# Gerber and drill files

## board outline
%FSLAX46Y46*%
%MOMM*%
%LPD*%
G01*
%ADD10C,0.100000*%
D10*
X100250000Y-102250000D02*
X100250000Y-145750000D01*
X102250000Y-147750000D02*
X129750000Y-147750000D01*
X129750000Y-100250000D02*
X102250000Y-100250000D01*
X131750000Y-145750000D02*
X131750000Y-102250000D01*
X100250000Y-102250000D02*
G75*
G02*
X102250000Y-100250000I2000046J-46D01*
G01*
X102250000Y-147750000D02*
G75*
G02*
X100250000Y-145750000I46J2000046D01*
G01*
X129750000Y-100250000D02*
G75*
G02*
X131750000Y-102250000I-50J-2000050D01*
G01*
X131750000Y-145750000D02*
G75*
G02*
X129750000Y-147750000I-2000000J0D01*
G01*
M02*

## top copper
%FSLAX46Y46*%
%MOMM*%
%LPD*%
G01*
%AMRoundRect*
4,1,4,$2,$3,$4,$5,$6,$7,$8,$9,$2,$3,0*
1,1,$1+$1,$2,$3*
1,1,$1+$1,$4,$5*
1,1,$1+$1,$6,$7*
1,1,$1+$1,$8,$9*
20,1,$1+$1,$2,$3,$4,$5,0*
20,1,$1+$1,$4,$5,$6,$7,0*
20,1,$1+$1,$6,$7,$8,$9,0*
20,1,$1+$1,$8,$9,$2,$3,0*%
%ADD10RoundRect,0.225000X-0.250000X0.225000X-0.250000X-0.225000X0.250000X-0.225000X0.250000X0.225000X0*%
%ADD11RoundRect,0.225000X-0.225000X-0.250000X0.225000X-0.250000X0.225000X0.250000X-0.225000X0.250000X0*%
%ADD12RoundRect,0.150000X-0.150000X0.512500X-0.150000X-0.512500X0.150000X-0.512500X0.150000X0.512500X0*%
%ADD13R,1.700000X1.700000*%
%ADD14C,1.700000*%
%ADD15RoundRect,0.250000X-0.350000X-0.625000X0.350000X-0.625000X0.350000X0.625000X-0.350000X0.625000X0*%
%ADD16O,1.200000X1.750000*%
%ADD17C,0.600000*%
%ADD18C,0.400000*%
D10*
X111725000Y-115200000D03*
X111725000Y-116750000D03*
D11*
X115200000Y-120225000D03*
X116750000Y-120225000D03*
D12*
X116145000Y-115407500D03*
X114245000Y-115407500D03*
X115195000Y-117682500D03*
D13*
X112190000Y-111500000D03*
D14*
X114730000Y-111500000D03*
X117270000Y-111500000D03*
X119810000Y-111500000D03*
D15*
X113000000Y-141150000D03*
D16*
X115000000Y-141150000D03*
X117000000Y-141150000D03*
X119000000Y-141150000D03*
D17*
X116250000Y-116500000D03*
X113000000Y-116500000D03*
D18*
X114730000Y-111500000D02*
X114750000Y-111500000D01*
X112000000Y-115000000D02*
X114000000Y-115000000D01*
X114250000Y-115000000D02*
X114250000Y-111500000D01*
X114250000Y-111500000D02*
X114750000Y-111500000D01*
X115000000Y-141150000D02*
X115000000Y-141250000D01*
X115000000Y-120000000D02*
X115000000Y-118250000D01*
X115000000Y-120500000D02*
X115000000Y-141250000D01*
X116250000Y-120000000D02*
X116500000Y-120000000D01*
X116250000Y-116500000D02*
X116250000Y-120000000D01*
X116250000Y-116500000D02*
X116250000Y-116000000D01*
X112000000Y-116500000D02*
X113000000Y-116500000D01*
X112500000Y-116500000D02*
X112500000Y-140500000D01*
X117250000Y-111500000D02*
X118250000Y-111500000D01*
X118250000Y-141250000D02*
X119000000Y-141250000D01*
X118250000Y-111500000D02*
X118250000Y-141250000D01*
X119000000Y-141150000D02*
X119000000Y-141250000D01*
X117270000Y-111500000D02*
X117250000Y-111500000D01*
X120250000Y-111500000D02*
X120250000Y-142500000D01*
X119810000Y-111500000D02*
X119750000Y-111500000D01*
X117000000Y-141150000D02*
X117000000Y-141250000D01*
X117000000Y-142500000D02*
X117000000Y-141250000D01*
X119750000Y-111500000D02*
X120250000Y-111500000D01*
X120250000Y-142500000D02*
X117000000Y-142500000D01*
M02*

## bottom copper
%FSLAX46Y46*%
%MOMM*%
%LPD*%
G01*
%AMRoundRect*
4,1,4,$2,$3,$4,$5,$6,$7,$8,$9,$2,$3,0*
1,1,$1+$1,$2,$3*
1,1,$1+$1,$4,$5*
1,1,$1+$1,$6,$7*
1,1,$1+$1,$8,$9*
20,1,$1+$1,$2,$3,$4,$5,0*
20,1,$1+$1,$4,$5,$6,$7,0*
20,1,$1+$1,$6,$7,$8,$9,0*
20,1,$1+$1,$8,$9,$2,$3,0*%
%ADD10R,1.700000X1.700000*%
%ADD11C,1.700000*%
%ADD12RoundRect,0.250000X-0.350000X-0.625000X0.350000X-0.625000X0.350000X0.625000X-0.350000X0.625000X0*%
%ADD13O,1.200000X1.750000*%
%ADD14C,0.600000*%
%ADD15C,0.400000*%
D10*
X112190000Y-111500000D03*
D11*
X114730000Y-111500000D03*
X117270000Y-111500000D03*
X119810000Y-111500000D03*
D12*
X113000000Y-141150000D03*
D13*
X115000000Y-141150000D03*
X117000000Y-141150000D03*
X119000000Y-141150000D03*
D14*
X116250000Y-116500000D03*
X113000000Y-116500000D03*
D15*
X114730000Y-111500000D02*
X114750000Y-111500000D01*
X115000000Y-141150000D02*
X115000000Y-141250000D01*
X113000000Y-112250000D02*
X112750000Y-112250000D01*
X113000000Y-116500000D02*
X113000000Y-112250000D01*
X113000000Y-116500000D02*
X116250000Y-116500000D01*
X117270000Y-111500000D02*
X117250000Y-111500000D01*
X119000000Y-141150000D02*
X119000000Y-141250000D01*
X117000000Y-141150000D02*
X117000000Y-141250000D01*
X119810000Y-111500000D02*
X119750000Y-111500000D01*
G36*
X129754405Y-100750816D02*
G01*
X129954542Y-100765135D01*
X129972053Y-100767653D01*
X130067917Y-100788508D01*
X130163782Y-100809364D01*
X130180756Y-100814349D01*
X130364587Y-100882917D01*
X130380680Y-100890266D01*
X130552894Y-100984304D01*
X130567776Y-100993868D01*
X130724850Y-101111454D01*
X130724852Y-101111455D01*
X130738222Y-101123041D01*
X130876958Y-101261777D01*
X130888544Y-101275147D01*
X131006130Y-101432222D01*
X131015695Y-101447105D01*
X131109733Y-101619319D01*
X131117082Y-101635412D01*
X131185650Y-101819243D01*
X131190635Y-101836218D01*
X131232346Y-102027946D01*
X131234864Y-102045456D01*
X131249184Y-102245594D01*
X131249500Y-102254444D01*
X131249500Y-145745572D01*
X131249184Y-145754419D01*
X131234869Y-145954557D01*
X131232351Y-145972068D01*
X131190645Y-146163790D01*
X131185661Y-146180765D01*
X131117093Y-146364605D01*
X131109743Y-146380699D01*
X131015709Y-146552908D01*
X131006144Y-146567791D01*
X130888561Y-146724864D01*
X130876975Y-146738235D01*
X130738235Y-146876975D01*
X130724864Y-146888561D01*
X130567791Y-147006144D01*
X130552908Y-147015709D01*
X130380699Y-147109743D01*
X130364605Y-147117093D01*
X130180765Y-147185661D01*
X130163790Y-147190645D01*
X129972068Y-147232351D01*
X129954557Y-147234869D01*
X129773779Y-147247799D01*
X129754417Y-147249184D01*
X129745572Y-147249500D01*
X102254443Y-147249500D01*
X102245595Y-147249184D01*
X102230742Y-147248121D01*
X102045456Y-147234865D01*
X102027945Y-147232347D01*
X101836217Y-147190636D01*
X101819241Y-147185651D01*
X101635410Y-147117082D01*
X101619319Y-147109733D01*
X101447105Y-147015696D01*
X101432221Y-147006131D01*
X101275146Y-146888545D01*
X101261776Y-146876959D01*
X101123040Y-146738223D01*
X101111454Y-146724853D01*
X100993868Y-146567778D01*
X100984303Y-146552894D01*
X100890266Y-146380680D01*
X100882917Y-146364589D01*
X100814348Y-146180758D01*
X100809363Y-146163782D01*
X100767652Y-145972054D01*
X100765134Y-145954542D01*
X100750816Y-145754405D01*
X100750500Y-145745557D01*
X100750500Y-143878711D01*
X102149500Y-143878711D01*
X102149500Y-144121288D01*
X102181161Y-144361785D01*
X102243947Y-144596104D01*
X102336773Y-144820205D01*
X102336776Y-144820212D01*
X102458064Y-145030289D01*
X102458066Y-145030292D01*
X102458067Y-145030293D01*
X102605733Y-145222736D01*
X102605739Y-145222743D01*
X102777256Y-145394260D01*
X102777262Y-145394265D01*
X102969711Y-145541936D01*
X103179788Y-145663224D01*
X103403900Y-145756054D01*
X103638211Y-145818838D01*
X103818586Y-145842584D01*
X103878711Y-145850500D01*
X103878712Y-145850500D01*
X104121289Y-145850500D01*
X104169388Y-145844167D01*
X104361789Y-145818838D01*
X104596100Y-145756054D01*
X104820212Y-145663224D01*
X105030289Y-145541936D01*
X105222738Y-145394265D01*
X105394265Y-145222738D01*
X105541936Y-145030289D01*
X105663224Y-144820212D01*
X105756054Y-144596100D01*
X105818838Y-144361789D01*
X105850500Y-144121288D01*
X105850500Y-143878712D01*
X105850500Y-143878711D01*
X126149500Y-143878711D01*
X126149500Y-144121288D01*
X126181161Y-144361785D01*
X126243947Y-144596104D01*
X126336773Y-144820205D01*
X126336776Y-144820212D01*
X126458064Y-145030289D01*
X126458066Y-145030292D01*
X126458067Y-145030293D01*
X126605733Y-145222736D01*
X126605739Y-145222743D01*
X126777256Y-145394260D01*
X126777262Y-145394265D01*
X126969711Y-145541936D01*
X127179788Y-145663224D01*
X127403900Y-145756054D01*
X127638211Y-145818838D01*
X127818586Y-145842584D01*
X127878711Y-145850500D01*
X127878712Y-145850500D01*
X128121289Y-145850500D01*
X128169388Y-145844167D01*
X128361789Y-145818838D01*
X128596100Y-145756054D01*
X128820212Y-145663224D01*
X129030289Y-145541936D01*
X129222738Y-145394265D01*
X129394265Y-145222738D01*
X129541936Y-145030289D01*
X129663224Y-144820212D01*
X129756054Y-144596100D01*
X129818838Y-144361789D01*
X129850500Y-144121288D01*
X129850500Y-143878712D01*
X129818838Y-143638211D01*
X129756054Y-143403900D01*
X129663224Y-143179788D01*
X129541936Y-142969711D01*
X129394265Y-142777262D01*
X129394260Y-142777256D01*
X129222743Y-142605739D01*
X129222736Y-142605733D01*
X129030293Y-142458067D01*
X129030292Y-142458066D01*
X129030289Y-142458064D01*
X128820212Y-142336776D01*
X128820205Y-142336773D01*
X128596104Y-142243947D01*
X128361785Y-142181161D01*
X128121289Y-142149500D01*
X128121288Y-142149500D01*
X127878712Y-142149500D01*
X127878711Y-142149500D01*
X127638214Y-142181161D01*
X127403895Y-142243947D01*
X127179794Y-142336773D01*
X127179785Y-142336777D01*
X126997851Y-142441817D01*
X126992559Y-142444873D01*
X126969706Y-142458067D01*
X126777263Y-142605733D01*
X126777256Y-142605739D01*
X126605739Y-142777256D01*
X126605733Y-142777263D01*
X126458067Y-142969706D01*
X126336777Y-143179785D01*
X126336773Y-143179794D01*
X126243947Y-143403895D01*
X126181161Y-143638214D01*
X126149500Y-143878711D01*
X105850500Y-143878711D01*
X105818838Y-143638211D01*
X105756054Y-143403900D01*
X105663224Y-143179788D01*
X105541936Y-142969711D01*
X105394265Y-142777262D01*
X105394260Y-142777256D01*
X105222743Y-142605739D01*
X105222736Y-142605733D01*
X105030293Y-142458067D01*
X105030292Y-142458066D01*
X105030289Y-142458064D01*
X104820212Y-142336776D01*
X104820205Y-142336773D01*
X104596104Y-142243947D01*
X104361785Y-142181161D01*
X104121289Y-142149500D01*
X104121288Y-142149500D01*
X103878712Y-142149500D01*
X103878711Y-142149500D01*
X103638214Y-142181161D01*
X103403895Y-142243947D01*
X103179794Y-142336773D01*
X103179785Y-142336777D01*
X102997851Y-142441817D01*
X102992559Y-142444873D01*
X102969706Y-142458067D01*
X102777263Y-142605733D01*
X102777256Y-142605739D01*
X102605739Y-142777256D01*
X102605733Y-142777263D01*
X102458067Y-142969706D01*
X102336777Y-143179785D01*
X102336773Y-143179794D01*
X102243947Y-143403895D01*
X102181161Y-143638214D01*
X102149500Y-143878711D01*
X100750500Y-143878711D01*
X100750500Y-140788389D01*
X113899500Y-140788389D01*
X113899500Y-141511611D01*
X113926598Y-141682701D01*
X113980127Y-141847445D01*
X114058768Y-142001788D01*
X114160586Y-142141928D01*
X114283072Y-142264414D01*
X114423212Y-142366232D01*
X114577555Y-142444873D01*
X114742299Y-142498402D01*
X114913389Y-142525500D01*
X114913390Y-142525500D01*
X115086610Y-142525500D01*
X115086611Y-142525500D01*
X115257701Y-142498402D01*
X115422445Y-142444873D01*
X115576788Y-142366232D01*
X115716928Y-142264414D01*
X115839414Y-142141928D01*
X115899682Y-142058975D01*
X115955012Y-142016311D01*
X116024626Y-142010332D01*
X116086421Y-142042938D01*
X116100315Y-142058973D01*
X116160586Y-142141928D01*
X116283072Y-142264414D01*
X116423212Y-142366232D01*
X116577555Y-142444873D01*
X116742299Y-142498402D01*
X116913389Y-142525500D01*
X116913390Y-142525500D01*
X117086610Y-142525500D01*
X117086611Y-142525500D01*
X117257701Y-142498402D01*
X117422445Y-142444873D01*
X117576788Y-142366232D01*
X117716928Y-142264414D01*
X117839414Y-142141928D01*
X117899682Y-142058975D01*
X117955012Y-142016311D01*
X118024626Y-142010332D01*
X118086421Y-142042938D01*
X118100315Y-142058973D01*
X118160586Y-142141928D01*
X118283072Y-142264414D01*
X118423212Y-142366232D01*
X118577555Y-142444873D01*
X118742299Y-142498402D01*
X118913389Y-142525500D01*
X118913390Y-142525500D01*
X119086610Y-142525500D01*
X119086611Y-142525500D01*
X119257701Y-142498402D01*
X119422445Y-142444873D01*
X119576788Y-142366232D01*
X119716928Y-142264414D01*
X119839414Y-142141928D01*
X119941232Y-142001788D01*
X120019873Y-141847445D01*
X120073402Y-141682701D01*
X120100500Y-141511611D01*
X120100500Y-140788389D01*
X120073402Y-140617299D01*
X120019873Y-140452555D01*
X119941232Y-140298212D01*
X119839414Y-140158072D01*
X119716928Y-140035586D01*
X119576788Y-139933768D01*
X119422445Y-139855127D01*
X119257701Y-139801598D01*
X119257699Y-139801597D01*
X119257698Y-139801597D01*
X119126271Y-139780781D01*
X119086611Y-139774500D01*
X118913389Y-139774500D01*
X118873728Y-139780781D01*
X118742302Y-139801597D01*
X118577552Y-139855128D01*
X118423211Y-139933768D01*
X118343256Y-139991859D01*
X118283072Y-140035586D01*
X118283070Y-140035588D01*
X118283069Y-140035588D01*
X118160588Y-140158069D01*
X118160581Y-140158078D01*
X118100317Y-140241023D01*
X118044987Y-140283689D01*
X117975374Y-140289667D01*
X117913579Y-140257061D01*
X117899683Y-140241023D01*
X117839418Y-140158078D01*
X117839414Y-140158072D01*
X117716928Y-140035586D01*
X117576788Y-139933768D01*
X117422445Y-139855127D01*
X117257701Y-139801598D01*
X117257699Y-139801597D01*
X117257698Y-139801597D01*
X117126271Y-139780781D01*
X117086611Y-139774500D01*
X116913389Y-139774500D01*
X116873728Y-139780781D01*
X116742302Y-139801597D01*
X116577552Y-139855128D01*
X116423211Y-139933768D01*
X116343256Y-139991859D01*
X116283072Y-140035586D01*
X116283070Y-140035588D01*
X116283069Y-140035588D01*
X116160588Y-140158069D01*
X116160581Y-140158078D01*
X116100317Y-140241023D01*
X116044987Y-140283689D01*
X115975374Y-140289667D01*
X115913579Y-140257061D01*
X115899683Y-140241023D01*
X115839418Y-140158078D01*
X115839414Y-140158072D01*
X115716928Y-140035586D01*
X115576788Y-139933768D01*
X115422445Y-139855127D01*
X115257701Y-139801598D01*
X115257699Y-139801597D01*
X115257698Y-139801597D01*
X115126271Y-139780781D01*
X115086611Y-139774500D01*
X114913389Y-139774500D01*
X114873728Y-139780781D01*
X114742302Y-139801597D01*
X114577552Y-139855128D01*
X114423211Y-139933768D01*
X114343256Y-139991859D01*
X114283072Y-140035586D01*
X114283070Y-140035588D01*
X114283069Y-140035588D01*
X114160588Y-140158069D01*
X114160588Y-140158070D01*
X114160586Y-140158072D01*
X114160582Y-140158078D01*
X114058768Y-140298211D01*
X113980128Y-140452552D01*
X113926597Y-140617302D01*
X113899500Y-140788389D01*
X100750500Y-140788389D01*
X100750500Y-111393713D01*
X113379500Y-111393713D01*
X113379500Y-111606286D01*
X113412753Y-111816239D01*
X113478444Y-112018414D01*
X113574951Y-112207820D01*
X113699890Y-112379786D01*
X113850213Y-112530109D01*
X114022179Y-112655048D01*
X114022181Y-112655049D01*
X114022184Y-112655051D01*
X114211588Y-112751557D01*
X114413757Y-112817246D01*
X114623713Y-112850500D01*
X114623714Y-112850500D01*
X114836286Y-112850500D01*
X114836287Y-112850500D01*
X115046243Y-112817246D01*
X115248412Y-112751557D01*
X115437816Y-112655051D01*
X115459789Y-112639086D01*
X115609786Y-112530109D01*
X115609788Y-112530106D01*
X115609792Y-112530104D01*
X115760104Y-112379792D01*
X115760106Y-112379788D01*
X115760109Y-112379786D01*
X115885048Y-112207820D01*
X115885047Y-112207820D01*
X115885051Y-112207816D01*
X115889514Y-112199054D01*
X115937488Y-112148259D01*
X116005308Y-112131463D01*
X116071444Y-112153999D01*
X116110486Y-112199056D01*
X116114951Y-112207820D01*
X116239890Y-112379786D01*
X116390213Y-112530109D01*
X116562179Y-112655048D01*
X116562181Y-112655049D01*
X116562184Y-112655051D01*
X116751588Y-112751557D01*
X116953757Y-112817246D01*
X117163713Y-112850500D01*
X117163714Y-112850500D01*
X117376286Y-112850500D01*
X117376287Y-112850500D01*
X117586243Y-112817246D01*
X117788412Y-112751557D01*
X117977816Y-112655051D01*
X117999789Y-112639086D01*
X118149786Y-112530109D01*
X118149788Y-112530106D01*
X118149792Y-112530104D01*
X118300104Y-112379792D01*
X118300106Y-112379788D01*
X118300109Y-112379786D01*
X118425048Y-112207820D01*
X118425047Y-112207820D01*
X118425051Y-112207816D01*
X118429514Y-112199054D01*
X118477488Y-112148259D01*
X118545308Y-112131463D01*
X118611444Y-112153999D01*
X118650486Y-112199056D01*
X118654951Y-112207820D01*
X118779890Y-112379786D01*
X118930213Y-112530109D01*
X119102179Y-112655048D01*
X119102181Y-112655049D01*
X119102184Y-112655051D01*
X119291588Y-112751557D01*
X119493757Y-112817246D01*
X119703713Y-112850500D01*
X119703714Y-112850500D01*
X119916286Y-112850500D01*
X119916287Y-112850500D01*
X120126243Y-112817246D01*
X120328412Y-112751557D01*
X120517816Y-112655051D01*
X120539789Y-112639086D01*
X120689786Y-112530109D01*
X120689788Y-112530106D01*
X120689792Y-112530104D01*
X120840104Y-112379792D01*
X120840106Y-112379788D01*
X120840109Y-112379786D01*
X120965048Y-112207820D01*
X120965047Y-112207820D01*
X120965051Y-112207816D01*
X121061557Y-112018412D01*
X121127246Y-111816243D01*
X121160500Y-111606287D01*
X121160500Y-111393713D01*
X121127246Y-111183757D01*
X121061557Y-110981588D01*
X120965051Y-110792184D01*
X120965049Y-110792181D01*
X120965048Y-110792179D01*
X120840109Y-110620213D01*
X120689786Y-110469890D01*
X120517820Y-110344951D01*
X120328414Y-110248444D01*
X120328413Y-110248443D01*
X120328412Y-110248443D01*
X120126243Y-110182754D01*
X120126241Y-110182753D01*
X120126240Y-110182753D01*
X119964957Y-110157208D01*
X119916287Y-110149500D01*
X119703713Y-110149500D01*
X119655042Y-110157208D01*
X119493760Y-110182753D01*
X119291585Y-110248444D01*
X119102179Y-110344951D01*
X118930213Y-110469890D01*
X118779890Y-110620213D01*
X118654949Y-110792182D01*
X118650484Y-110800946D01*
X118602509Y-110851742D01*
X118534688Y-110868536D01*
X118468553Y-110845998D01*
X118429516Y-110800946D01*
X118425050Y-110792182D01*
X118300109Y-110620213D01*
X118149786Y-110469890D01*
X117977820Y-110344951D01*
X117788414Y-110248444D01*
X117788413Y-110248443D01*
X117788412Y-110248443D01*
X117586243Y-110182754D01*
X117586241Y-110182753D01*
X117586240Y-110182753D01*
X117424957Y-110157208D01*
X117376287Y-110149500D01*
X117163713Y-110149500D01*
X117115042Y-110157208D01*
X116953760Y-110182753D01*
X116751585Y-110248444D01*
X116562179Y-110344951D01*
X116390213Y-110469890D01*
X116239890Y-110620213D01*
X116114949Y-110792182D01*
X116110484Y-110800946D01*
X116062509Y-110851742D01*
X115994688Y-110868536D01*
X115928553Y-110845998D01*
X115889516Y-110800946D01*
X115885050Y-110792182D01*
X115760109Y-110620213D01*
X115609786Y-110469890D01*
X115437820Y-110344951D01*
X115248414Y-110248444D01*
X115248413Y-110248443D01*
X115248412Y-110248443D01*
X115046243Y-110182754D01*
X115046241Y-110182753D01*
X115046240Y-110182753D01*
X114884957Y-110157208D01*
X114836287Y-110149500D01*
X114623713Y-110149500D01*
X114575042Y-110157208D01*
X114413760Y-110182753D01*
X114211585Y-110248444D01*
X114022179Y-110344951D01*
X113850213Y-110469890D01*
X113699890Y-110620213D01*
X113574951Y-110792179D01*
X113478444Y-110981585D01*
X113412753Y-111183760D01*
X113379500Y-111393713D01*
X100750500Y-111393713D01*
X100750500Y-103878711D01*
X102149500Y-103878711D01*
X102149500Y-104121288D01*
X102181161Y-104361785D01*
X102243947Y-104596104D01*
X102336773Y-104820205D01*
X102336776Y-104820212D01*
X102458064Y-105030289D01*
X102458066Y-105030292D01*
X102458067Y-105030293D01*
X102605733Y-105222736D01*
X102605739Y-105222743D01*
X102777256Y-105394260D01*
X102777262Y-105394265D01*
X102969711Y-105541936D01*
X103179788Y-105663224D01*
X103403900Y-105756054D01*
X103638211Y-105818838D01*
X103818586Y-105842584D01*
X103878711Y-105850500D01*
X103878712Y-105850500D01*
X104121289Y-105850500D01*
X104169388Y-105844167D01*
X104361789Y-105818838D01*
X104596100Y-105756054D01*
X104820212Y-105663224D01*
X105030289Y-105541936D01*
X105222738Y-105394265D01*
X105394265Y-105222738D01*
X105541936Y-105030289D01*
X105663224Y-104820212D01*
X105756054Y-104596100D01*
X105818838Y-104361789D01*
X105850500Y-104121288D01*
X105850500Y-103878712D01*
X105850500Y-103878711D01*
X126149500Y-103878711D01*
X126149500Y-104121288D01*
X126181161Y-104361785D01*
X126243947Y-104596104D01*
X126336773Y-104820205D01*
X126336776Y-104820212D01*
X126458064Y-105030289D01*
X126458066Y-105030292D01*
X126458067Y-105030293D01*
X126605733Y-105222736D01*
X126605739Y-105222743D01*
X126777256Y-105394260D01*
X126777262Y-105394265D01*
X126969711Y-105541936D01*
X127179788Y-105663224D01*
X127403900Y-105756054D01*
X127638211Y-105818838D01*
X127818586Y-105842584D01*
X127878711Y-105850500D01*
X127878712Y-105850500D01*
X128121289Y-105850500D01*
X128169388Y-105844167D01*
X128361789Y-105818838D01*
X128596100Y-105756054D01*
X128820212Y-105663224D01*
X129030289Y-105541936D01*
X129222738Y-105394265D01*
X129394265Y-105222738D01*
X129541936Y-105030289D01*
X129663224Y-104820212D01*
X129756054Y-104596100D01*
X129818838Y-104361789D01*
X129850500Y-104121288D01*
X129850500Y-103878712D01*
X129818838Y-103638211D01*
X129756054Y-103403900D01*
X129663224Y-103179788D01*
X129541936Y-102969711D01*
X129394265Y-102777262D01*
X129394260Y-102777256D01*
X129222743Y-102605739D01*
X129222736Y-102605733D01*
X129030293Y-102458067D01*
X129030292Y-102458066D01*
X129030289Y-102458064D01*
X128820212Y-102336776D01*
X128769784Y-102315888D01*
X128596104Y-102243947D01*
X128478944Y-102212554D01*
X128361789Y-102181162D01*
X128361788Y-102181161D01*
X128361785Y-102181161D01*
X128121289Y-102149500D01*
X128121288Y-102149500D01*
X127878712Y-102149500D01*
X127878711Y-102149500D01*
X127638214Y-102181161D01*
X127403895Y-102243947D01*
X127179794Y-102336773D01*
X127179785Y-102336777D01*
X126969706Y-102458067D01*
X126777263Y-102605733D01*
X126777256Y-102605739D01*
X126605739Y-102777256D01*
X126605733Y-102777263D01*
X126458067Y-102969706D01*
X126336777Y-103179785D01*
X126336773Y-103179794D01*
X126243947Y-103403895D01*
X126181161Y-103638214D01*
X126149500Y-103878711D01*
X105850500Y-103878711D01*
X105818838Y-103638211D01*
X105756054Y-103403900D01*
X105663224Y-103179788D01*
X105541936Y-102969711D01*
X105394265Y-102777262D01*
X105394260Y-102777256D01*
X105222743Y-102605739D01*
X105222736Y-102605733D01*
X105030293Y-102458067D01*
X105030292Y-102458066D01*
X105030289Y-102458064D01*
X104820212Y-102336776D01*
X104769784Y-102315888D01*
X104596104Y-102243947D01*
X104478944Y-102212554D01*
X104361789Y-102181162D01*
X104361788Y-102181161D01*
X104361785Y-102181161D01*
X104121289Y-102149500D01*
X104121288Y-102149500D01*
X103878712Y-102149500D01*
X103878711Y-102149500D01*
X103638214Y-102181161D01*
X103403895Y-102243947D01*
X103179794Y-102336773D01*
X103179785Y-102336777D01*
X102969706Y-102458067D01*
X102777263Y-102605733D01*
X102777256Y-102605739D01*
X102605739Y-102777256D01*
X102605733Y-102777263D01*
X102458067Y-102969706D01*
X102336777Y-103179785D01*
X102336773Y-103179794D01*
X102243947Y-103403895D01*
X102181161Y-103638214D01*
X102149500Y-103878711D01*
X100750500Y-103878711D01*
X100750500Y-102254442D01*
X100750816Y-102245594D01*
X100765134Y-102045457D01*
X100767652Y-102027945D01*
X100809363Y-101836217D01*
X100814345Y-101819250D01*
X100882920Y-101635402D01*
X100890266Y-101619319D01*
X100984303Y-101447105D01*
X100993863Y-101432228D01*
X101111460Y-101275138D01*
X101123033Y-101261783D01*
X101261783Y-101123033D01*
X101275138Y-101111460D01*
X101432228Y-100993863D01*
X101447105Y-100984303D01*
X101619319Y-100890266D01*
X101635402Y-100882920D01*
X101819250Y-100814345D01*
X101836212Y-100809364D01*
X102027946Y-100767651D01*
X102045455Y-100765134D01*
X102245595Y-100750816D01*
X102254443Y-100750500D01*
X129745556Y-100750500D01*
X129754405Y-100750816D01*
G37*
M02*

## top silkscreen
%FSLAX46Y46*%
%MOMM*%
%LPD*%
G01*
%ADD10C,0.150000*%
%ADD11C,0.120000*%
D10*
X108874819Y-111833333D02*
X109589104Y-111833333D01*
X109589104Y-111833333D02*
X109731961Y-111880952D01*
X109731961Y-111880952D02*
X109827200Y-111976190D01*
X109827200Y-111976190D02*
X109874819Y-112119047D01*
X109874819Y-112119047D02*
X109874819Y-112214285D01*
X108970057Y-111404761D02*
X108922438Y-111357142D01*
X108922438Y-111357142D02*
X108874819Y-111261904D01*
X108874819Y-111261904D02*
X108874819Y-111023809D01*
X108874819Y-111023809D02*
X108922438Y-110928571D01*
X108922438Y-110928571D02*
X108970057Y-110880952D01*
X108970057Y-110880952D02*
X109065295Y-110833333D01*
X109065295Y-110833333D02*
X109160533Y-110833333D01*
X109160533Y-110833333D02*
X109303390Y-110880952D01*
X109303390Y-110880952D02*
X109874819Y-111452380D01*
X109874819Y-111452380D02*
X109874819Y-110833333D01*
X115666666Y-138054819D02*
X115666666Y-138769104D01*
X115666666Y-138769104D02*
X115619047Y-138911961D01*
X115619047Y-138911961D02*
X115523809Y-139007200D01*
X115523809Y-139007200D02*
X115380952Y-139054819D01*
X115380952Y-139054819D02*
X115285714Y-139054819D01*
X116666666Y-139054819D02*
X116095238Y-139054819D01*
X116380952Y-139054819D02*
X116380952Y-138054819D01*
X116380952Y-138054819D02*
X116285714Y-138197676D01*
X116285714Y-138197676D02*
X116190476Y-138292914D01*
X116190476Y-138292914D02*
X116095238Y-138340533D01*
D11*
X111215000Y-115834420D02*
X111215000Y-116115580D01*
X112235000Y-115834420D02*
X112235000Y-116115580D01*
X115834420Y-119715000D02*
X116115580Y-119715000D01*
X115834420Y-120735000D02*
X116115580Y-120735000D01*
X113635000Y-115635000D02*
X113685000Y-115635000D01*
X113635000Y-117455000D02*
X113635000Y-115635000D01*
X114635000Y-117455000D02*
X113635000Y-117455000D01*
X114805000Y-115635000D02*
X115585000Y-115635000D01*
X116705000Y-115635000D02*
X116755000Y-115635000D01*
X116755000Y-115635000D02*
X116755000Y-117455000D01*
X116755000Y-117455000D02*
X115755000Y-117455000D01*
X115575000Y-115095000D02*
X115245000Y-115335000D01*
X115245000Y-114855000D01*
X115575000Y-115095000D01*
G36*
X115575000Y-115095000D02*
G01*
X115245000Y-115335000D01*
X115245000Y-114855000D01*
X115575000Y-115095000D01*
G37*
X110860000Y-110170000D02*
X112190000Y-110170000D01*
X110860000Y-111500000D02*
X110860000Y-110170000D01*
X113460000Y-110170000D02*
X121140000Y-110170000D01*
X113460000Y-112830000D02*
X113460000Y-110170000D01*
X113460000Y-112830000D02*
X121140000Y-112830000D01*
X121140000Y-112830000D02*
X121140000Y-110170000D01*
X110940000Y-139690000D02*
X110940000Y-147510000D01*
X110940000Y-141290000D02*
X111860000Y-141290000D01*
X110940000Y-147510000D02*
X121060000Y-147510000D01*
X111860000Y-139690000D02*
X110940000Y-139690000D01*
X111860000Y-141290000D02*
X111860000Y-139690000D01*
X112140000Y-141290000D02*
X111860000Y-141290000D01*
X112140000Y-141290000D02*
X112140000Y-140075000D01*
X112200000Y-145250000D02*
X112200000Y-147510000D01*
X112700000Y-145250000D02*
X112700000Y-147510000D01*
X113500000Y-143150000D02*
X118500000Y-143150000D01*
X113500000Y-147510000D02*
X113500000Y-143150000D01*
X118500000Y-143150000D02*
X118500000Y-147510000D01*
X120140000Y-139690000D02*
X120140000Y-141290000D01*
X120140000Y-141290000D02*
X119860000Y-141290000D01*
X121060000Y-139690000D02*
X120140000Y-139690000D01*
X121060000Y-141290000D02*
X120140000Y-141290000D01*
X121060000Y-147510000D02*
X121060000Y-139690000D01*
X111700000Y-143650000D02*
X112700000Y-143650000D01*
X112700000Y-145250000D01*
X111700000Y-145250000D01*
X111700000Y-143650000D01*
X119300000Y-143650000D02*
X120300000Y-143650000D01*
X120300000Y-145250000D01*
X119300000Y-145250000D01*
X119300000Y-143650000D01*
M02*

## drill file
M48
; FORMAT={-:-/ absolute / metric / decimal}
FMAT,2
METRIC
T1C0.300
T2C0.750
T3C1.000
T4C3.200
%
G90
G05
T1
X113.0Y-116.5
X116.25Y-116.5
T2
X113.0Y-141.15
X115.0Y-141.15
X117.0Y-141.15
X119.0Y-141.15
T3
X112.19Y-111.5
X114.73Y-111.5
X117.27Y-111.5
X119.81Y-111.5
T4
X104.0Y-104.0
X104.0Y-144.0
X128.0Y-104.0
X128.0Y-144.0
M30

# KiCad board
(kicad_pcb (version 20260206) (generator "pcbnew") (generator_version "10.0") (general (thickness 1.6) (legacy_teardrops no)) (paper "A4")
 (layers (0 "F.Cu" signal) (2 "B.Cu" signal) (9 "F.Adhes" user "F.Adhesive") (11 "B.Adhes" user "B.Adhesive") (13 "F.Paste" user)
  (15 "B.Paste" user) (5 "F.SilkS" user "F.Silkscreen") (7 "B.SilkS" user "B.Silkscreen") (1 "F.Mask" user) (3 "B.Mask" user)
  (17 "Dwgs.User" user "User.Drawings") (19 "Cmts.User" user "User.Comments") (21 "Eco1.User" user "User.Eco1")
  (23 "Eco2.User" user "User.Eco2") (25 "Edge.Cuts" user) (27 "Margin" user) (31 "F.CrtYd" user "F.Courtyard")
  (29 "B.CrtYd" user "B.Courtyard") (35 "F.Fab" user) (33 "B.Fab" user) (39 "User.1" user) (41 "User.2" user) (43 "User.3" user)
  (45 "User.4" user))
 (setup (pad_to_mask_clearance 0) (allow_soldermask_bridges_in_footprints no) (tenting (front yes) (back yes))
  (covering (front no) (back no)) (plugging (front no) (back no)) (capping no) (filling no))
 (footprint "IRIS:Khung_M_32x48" (layer "F.Cu") (at 100 148)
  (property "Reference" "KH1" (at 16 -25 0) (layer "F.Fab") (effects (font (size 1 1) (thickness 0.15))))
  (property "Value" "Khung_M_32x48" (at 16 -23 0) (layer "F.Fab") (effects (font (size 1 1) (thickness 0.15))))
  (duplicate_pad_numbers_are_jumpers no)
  (fp_line (start 0.25 -45.75) (end 0.25 -2.25) (stroke (width 0.1) (type solid)) (layer "Edge.Cuts"))
  (fp_line (start 2.25 -0.25) (end 29.75 -0.25) (stroke (width 0.1) (type solid)) (layer "Edge.Cuts"))
  (fp_line (start 29.75 -47.75) (end 2.25 -47.75) (stroke (width 0.1) (type solid)) (layer "Edge.Cuts"))
  (fp_line (start 31.75 -2.25) (end 31.75 -45.75) (stroke (width 0.1) (type solid)) (layer "Edge.Cuts"))
  (fp_arc (start 0.25 -45.75) (mid 0.8358 -47.1642) (end 2.25 -47.75) (stroke (width 0.1) (type solid)) (layer "Edge.Cuts"))
  (fp_arc (start 2.25 -0.25) (mid 0.8358 -0.8358) (end 0.25 -2.25) (stroke (width 0.1) (type solid)) (layer "Edge.Cuts"))
  (fp_arc (start 29.75 -47.75) (mid 31.164199 -47.164199) (end 31.75 -45.75) (stroke (width 0.1) (type solid)) (layer "Edge.Cuts"))
  (fp_arc (start 31.75 -2.25) (mid 31.164214 -0.835786) (end 29.75 -0.25) (stroke (width 0.1) (type solid)) (layer "Edge.Cuts"))
  (pad "" np_thru_hole circle (at 4 -44) (size 3.2 3.2) (drill 3.2) (layers "*.Cu" "*.Mask"))
  (pad "" np_thru_hole circle (at 4 -4) (size 3.2 3.2) (drill 3.2) (layers "*.Cu" "*.Mask"))
  (pad "" np_thru_hole circle (at 28 -44) (size 3.2 3.2) (drill 3.2) (layers "*.Cu" "*.Mask"))
  (pad "" np_thru_hole circle (at 28 -4) (size 3.2 3.2) (drill 3.2) (layers "*.Cu" "*.Mask")))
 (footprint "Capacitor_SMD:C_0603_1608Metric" (layer "F.Cu") (at 111.725 115.975 -90)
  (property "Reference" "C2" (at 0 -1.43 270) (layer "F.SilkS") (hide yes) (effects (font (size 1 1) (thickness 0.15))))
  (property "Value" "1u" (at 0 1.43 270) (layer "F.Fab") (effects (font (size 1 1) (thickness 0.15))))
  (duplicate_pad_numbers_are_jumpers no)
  (fp_line (start -0.14058 0.51) (end 0.14058 0.51) (stroke (width 0.12) (type solid)) (layer "F.SilkS"))
  (fp_line (start -0.14058 -0.51) (end 0.14058 -0.51) (stroke (width 0.12) (type solid)) (layer "F.SilkS"))
  (pad "1" smd roundrect (at -0.775 0 270) (size 0.9 0.95) (layers "F.Cu" "F.Mask" "F.Paste") (roundrect_rratio 0.25) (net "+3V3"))
  (pad "2" smd roundrect (at 0.775 0 270) (size 0.9 0.95) (layers "F.Cu" "F.Mask" "F.Paste") (roundrect_rratio 0.25) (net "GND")))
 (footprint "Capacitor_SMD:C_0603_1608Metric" (layer "F.Cu") (at 115.975 120.225)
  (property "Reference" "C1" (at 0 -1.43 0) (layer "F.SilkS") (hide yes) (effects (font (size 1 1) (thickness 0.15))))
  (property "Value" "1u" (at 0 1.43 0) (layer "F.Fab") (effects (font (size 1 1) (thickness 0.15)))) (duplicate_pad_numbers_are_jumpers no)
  (fp_line (start -0.14058 -0.51) (end 0.14058 -0.51) (stroke (width 0.12) (type solid)) (layer "F.SilkS"))
  (fp_line (start -0.14058 0.51) (end 0.14058 0.51) (stroke (width 0.12) (type solid)) (layer "F.SilkS"))
  (pad "1" smd roundrect (at -0.775 0) (size 0.9 0.95) (layers "F.Cu" "F.Mask" "F.Paste") (roundrect_rratio 0.25) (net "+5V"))
  (pad "2" smd roundrect (at 0.775 0) (size 0.9 0.95) (layers "F.Cu" "F.Mask" "F.Paste") (roundrect_rratio 0.25) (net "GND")))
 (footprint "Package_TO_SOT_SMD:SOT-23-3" (layer "F.Cu") (at 115.195 116.545 -90)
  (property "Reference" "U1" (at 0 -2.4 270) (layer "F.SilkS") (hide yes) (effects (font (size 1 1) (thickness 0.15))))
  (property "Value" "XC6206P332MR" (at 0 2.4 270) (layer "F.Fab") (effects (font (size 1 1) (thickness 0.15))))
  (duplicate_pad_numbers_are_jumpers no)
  (fp_line (start -0.91 1.56) (end -0.91 1.51) (stroke (width 0.12) (type solid)) (layer "F.SilkS"))
  (fp_line (start 0.91 1.56) (end -0.91 1.56) (stroke (width 0.12) (type solid)) (layer "F.SilkS"))
  (fp_line (start 0.91 0.56) (end 0.91 1.56) (stroke (width 0.12) (type solid)) (layer "F.SilkS"))
  (fp_line (start -0.91 0.39) (end -0.91 -0.39) (stroke (width 0.12) (type solid)) (layer "F.SilkS"))
  (fp_line (start -0.91 -1.51) (end -0.91 -1.56) (stroke (width 0.12) (type solid)) (layer "F.SilkS"))
  (fp_line (start -0.91 -1.56) (end 0.91 -1.56) (stroke (width 0.12) (type solid)) (layer "F.SilkS"))
  (fp_line (start 0.91 -1.56) (end 0.91 -0.56) (stroke (width 0.12) (type solid)) (layer "F.SilkS"))
  (fp_poly (pts (xy -1.45 -0.38) (xy -1.21 -0.05) (xy -1.69 -0.05)) (stroke (width 0.12) (type solid)) (fill yes) (layer "F.SilkS"))
  (pad "1" smd roundrect (at -1.1375 -0.95 270) (size 1.325 0.6) (layers "F.Cu" "F.Mask" "F.Paste") (roundrect_rratio 0.25) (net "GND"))
  (pad "2" smd roundrect (at -1.1375 0.95 270) (size 1.325 0.6) (layers "F.Cu" "F.Mask" "F.Paste") (roundrect_rratio 0.25) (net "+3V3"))
  (pad "3" smd roundrect (at 1.1375 0 270) (size 1.325 0.6) (layers "F.Cu" "F.Mask" "F.Paste") (roundrect_rratio 0.25) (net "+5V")))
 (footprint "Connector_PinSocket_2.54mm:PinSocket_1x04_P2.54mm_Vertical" (layer "F.Cu") (at 112.19 111.5 90)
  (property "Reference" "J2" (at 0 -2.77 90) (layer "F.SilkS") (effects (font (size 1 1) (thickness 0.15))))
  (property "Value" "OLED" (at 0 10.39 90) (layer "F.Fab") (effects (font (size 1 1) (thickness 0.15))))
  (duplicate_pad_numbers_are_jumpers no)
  (fp_line (start 1.33 -1.33) (end 1.33 0) (stroke (width 0.12) (type solid)) (layer "F.SilkS"))
  (fp_line (start 0 -1.33) (end 1.33 -1.33) (stroke (width 0.12) (type solid)) (layer "F.SilkS"))
  (fp_line (start 1.33 1.27) (end 1.33 8.95) (stroke (width 0.12) (type solid)) (layer "F.SilkS"))
  (fp_line (start -1.33 1.27) (end 1.33 1.27) (stroke (width 0.12) (type solid)) (layer "F.SilkS"))
  (fp_line (start -1.33 1.27) (end -1.33 8.95) (stroke (width 0.12) (type solid)) (layer "F.SilkS"))
  (fp_line (start -1.33 8.95) (end 1.33 8.95) (stroke (width 0.12) (type solid)) (layer "F.SilkS"))
  (pad "1" thru_hole rect (at 0 0 90) (size 1.7 1.7) (drill 1) (layers "*.Cu" "*.Mask") (remove_unused_layers no) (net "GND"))
  (pad "2" thru_hole circle (at 0 2.54 90) (size 1.7 1.7) (drill 1) (layers "*.Cu" "*.Mask") (remove_unused_layers no) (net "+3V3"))
  (pad "3" thru_hole circle (at 0 5.08 90) (size 1.7 1.7) (drill 1) (layers "*.Cu" "*.Mask") (remove_unused_layers no) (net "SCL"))
  (pad "4" thru_hole circle (at 0 7.62 90) (size 1.7 1.7) (drill 1) (layers "*.Cu" "*.Mask") (remove_unused_layers no) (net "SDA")))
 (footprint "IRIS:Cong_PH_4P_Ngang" (layer "F.Cu") (at 113 141.15)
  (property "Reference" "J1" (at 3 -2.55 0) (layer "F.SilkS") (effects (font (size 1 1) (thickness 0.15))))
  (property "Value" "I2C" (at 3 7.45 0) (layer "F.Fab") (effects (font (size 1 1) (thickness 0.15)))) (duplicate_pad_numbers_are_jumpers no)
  (fp_line (start -2.06 -1.46) (end -2.06 6.36) (stroke (width 0.12) (type solid)) (layer "F.SilkS"))
  (fp_line (start -2.06 0.14) (end -1.14 0.14) (stroke (width 0.12) (type solid)) (layer "F.SilkS"))
  (fp_line (start -2.06 6.36) (end 8.06 6.36) (stroke (width 0.12) (type solid)) (layer "F.SilkS"))
  (fp_line (start -1.14 -1.46) (end -2.06 -1.46) (stroke (width 0.12) (type solid)) (layer "F.SilkS"))
  (fp_line (start -1.14 0.14) (end -1.14 -1.46) (stroke (width 0.12) (type solid)) (layer "F.SilkS"))
  (fp_line (start -0.86 0.14) (end -1.14 0.14) (stroke (width 0.12) (type solid)) (layer "F.SilkS"))
  (fp_line (start -0.86 0.14) (end -0.86 -1.075) (stroke (width 0.12) (type solid)) (layer "F.SilkS"))
  (fp_line (start -0.8 4.1) (end -0.8 6.36) (stroke (width 0.12) (type solid)) (layer "F.SilkS"))
  (fp_line (start -0.3 4.1) (end -0.3 6.36) (stroke (width 0.12) (type solid)) (layer "F.SilkS"))
  (fp_line (start 0.5 2) (end 5.5 2) (stroke (width 0.12) (type solid)) (layer "F.SilkS"))
  (fp_line (start 0.5 6.36) (end 0.5 2) (stroke (width 0.12) (type solid)) (layer "F.SilkS"))
  (fp_line (start 5.5 2) (end 5.5 6.36) (stroke (width 0.12) (type solid)) (layer "F.SilkS"))
  (fp_line (start 7.14 -1.46) (end 7.14 0.14) (stroke (width 0.12) (type solid)) (layer "F.SilkS"))
  (fp_line (start 7.14 0.14) (end 6.86 0.14) (stroke (width 0.12) (type solid)) (layer "F.SilkS"))
  (fp_line (start 8.06 -1.46) (end 7.14 -1.46) (stroke (width 0.12) (type solid)) (layer "F.SilkS"))
  (fp_line (start 8.06 0.14) (end 7.14 0.14) (stroke (width 0.12) (type solid)) (layer "F.SilkS"))
  (fp_line (start 8.06 6.36) (end 8.06 -1.46) (stroke (width 0.12) (type solid)) (layer "F.SilkS"))
  (fp_rect (start -1.3 2.5) (end -0.3 4.1) (stroke (width 0.12) (type solid)) (fill no) (layer "F.SilkS"))
  (fp_rect (start 6.3 2.5) (end 7.3 4.1) (stroke (width 0.12) (type solid)) (fill no) (layer "F.SilkS"))
  (pad "1" thru_hole roundrect (at 0 0) (size 1.2 1.75) (drill 0.75) (layers "*.Cu" "*.Mask") (remove_unused_layers no)
   (roundrect_rratio 0.208333) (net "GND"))
  (pad "2" thru_hole oval (at 2 0) (size 1.2 1.75) (drill 0.75) (layers "*.Cu" "*.Mask") (remove_unused_layers no) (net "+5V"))
  (pad "3" thru_hole oval (at 4 0) (size 1.2 1.75) (drill 0.75) (layers "*.Cu" "*.Mask") (remove_unused_layers no) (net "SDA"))
  (pad "4" thru_hole oval (at 6 0) (size 1.2 1.75) (drill 0.75) (layers "*.Cu" "*.Mask") (remove_unused_layers no) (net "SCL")))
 (segment (start 114.73 111.5) (end 114.75 111.5) (width 0.4) (layer "F.Cu") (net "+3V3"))
 (segment (start 112 115) (end 114 115) (width 0.4) (layer "F.Cu") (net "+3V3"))
 (segment (start 114.25 115) (end 114.25 111.5) (width 0.4) (layer "F.Cu") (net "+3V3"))
 (segment (start 114.25 111.5) (end 114.75 111.5) (width 0.4) (layer "F.Cu") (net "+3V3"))
 (segment (start 114.73 111.5) (end 114.75 111.5) (width 0.4) (layer "B.Cu") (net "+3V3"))
 (segment (start 115 141.15) (end 115 141.25) (width 0.4) (layer "F.Cu") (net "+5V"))
 (segment (start 115 120) (end 115 118.25) (width 0.4) (layer "F.Cu") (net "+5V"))
 (segment (start 115 120.5) (end 115 141.25) (width 0.4) (layer "F.Cu") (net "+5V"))
 (segment (start 115 141.15) (end 115 141.25) (width 0.4) (layer "B.Cu") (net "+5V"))
 (segment (start 116.25 120) (end 116.5 120) (width 0.4) (layer "F.Cu") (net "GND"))
 (segment (start 116.25 116.5) (end 116.25 120) (width 0.4) (layer "F.Cu") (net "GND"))
 (segment (start 116.25 116.5) (end 116.25 116) (width 0.4) (layer "F.Cu") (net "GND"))
 (segment (start 112 116.5) (end 113 116.5) (width 0.4) (layer "F.Cu") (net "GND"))
 (segment (start 112.5 116.5) (end 112.5 140.5) (width 0.4) (layer "F.Cu") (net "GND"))
 (via (at 116.25 116.5) (size 0.6) (drill 0.3) (layers "F.Cu" "B.Cu") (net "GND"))
 (via (at 113 116.5) (size 0.6) (drill 0.3) (layers "F.Cu" "B.Cu") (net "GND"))
 (segment (start 113 112.25) (end 112.75 112.25) (width 0.4) (layer "B.Cu") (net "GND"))
 (segment (start 113 116.5) (end 113 112.25) (width 0.4) (layer "B.Cu") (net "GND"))
 (segment (start 113 116.5) (end 116.25 116.5) (width 0.4) (layer "B.Cu") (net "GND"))
 (segment (start 117.25 111.5) (end 118.25 111.5) (width 0.4) (layer "F.Cu") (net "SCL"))
 (segment (start 118.25 141.25) (end 119 141.25) (width 0.4) (layer "F.Cu") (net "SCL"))
 (segment (start 118.25 111.5) (end 118.25 141.25) (width 0.4) (layer "F.Cu") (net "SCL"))
 (segment (start 119 141.15) (end 119 141.25) (width 0.4) (layer "F.Cu") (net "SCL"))
 (segment (start 117.27 111.5) (end 117.25 111.5) (width 0.4) (layer "F.Cu") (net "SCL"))
 (segment (start 117.27 111.5) (end 117.25 111.5) (width 0.4) (layer "B.Cu") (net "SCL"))
 (segment (start 119 141.15) (end 119 141.25) (width 0.4) (layer "B.Cu") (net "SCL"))
 (segment (start 120.25 111.5) (end 120.25 142.5) (width 0.4) (layer "F.Cu") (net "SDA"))
 (segment (start 119.81 111.5) (end 119.75 111.5) (width 0.4) (layer "F.Cu") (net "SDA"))
 (segment (start 117 141.15) (end 117 141.25) (width 0.4) (layer "F.Cu") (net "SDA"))
 (segment (start 117 142.5) (end 117 141.25) (width 0.4) (layer "F.Cu") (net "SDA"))
 (segment (start 119.75 111.5) (end 120.25 111.5) (width 0.4) (layer "F.Cu") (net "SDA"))
 (segment (start 120.25 142.5) (end 117 142.5) (width 0.4) (layer "F.Cu") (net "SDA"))
 (segment (start 117 141.15) (end 117 141.25) (width 0.4) (layer "B.Cu") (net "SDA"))
 (segment (start 119.81 111.5) (end 119.75 111.5) (width 0.4) (layer "B.Cu") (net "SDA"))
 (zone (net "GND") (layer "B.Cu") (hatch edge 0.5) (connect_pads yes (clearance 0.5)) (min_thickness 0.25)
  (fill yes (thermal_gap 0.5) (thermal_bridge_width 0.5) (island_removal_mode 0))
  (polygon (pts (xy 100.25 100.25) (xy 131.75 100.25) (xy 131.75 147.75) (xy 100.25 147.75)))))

